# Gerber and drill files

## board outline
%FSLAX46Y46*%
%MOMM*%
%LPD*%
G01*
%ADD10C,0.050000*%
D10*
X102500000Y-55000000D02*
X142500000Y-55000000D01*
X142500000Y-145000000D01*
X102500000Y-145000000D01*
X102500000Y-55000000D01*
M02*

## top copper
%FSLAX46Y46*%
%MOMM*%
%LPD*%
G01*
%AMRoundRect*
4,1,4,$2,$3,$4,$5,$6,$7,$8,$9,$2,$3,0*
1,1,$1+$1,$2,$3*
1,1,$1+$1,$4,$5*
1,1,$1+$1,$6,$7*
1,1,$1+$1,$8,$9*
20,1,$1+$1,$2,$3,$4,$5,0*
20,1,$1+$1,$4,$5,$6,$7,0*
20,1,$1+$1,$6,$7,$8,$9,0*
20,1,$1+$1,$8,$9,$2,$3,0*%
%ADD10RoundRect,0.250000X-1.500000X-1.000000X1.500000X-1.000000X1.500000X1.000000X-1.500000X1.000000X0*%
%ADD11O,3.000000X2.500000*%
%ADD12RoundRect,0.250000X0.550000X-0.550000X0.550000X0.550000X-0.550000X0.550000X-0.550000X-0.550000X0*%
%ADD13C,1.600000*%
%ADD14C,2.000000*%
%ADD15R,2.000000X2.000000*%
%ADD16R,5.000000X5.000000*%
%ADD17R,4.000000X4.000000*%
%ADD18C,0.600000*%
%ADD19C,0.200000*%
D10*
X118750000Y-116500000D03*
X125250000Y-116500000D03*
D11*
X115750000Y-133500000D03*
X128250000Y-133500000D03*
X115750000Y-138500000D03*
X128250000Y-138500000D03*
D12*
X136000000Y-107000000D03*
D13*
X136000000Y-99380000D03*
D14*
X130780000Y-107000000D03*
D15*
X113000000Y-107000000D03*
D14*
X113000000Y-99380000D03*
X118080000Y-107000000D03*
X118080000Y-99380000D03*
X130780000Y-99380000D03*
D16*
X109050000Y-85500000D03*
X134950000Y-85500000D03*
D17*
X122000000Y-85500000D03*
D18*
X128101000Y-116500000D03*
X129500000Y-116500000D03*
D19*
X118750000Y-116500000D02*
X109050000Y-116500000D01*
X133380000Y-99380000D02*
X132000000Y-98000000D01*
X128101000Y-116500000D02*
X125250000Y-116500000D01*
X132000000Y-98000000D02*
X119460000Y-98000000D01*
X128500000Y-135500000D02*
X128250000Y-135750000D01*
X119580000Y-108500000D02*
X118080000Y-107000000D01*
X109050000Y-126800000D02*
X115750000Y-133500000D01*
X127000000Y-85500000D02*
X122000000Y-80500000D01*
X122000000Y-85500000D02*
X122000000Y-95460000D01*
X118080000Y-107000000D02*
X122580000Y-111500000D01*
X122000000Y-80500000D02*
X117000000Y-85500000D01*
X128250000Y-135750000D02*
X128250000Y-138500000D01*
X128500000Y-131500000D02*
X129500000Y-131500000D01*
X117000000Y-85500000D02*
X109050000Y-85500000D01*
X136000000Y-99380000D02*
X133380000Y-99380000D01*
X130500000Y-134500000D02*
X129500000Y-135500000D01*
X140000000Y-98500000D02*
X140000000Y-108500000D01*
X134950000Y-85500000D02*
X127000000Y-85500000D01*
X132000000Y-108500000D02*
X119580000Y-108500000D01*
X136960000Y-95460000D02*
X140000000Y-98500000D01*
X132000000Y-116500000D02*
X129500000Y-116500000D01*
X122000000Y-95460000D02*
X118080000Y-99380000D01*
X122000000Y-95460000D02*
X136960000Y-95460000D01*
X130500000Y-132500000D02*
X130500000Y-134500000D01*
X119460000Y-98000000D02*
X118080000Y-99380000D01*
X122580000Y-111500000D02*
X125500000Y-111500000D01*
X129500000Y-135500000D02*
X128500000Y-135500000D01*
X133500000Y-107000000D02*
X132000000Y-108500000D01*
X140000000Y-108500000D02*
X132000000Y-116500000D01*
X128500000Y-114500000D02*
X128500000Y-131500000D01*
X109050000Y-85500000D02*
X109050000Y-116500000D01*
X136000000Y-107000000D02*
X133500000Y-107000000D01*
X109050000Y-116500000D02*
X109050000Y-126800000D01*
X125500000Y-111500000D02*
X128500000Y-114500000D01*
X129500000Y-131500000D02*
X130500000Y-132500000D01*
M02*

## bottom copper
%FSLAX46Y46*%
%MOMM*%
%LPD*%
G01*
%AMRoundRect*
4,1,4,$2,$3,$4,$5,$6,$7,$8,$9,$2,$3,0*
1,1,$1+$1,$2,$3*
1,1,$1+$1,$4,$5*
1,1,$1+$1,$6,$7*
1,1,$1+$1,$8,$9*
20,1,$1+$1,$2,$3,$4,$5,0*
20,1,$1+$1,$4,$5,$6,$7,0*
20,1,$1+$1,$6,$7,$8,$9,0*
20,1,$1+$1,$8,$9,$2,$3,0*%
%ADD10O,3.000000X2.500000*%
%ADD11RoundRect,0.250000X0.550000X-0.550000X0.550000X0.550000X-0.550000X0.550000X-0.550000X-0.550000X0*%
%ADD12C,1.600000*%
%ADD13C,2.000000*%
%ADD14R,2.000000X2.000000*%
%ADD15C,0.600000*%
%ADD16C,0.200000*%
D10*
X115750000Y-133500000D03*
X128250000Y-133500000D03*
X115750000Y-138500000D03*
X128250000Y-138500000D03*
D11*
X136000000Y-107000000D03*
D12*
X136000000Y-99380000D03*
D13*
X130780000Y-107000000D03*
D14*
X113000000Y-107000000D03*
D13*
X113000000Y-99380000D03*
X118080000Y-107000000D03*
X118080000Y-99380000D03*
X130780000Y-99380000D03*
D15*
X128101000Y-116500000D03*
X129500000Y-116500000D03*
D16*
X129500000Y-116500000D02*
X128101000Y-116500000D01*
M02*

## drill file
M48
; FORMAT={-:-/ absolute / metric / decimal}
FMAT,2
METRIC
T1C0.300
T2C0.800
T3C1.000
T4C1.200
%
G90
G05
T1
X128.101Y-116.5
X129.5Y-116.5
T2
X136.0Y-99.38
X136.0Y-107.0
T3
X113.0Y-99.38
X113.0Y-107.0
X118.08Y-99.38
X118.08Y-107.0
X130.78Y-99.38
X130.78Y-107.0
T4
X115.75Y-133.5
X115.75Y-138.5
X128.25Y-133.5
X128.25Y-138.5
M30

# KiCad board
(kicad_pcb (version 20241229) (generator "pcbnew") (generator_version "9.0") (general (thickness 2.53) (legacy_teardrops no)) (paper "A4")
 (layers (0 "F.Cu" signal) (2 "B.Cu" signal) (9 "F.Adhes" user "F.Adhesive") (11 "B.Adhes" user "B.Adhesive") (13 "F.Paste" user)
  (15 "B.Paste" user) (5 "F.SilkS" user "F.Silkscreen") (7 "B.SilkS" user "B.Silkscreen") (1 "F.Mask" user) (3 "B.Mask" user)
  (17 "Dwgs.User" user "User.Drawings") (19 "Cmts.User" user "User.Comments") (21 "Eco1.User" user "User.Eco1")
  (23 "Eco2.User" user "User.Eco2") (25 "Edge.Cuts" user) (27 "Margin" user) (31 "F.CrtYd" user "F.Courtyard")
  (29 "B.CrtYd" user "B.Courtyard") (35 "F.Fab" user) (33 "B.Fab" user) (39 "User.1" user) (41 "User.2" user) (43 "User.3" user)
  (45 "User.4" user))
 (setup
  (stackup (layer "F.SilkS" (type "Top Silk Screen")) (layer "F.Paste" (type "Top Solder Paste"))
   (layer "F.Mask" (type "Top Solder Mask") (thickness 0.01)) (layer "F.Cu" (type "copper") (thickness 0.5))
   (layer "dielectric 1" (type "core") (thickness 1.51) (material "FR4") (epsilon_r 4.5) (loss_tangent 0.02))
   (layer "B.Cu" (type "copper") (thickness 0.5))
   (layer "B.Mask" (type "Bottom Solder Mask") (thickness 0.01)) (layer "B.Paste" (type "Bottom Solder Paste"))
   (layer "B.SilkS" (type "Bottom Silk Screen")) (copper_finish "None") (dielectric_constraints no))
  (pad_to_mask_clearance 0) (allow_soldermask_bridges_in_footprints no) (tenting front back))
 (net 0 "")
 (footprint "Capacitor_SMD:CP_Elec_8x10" (layer "F.Cu") (at 122 116.5)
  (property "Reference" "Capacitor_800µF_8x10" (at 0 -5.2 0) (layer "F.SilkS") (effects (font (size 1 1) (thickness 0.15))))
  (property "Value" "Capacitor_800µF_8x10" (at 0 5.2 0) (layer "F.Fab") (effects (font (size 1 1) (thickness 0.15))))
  (pad "1" smd roundrect (at -3.25 0) (size 3.5 2.5) (layers "F.Cu" "F.Mask" "F.Paste") (roundrect_rratio 0.1))
  (pad "2" smd roundrect (at 3.25 0) (size 3.5 2.5) (layers "F.Cu" "F.Mask" "F.Paste") (roundrect_rratio 0.1)))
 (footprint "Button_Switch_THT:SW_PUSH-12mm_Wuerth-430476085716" (layer "F.Cu") (at 115.75 133.5)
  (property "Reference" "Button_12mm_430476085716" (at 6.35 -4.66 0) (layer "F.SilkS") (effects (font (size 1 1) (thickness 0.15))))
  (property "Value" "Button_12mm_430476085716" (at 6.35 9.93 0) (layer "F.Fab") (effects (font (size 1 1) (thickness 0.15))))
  (pad "1" thru_hole oval (at 0 0) (size 3 2.5) (drill 1.2) (layers "*.Cu" "*.Mask") (remove_unused_layers no))
  (pad "1" thru_hole oval (at 12.5 0) (size 3 2.5) (drill 1.2) (layers "*.Cu" "*.Mask") (remove_unused_layers no))
  (pad "2" thru_hole oval (at 0 5) (size 3 2.5) (drill 1.2) (layers "*.Cu" "*.Mask") (remove_unused_layers no))
  (pad "2" thru_hole oval (at 12.5 5) (size 3 2.5) (drill 1.2) (layers "*.Cu" "*.Mask") (remove_unused_layers no)))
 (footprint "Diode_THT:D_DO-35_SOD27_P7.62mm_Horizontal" (layer "F.Cu") (at 136 107 90)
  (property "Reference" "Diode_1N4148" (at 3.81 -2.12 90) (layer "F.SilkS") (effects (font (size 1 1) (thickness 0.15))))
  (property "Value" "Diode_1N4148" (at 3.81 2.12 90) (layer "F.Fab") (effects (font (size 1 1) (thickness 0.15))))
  (pad "1" thru_hole roundrect (at 0 0 90) (size 1.6 1.6) (drill 0.8) (layers "*.Cu" "*.Mask") (remove_unused_layers no)
   (roundrect_rratio 0.15625))
  (pad "2" thru_hole circle (at 7.62 0 90) (size 1.6 1.6) (drill 0.8) (layers "*.Cu" "*.Mask") (remove_unused_layers no)))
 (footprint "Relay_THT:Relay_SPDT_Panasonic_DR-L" (layer "F.Cu") (at 113 107)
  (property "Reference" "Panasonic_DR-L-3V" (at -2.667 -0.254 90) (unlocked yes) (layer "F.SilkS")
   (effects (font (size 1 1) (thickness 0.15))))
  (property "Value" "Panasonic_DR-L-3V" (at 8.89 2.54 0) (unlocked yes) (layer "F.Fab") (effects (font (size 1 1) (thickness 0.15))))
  (pad "11" thru_hole circle (at 17.78 0 180) (size 2 2) (drill 1) (layers "*.Cu" "*.Mask") (remove_unused_layers no))
  (pad "12" thru_hole rect (at 0 0 180) (size 2 2) (drill 1) (layers "*.Cu" "*.Mask") (remove_unused_layers no))
  (pad "14" thru_hole circle (at 0 -7.62 180) (size 2 2) (drill 1) (layers "*.Cu" "*.Mask") (remove_unused_layers no))
  (pad "A1" thru_hole circle (at 5.08 0 180) (size 2 2) (drill 1) (layers "*.Cu" "*.Mask") (remove_unused_layers no))
  (pad "A2" thru_hole circle (at 5.08 -7.62 180) (size 2 2) (drill 1) (layers "*.Cu" "*.Mask") (remove_unused_layers no))
  (pad "PE" thru_hole circle (at 17.78 -7.62 180) (size 2 2) (drill 1) (layers "*.Cu" "*.Mask") (remove_unused_layers no)))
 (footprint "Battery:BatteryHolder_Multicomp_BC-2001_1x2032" (layer "F.Cu") (at 122 85.5)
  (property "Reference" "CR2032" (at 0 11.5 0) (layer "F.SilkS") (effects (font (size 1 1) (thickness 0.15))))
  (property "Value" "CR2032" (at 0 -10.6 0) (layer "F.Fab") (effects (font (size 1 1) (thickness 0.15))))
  (pad "1" smd rect (at -12.95 0) (size 5 5) (layers "F.Cu" "F.Mask" "F.Paste"))
  (pad "1" smd rect (at 12.95 0) (size 5 5) (layers "F.Cu" "F.Mask" "F.Paste"))
  (pad "2" smd rect (at 0 0) (size 4 4) (layers "F.Cu" "F.Mask" "F.Paste"))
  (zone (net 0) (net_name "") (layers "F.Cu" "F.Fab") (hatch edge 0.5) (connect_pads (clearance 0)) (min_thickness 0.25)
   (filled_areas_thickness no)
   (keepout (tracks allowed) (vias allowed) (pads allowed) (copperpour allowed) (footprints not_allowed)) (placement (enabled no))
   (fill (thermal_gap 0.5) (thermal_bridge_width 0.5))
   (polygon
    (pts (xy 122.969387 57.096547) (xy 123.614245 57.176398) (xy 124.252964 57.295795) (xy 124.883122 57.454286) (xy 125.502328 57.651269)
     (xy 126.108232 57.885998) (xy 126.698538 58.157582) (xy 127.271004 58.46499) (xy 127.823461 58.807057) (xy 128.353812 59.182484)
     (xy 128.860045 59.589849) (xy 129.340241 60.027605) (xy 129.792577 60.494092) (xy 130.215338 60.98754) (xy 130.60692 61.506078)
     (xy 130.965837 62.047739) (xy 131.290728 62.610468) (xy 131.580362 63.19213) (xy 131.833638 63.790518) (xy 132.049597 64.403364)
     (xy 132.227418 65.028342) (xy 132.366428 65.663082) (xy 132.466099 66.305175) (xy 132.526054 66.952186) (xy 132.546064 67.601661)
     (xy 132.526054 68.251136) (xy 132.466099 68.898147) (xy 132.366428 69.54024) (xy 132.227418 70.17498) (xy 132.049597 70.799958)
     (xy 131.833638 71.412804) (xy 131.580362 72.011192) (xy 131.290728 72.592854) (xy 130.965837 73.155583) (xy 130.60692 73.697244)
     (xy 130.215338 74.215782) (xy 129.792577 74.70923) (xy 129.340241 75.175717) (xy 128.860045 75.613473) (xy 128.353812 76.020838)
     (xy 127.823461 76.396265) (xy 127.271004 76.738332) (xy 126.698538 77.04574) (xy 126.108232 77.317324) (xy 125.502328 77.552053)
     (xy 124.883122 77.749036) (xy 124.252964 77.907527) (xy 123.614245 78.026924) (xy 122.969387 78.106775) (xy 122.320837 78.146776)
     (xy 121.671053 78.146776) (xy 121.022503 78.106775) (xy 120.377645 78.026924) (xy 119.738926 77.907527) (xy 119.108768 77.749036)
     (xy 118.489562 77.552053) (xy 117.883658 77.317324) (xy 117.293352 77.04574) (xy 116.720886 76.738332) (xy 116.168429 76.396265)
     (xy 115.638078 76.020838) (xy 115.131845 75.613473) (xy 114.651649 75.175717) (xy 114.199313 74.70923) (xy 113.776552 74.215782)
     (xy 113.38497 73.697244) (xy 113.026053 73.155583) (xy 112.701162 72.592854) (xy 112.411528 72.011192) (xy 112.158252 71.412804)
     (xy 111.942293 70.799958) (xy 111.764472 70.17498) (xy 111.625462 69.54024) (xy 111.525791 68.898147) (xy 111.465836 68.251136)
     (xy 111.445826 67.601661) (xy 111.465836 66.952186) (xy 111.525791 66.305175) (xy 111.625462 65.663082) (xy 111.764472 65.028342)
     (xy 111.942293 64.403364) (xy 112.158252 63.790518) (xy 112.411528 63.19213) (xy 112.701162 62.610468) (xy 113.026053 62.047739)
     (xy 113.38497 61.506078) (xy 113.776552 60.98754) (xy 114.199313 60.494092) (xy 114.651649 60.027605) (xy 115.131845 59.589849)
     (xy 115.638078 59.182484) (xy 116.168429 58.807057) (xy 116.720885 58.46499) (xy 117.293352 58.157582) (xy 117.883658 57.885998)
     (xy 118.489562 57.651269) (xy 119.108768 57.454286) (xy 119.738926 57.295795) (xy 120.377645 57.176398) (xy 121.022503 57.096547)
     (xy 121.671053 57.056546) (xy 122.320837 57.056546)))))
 (gr_rect (start 102.5 55) (end 142.5 145) (stroke (width 0.05) (type default)) (fill no) (layer "Edge.Cuts"))
 (segment (start 118.75 116.5) (end 109.05 116.5) (width 0.2) (layer "F.Cu") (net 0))
 (segment (start 133.38 99.38) (end 132 98) (width 0.2) (layer "F.Cu") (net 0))
 (segment (start 128.101 116.5) (end 125.25 116.5) (width 0.2) (layer "F.Cu") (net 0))
 (segment (start 132 98) (end 119.46 98) (width 0.2) (layer "F.Cu") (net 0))
 (segment (start 128.5 135.5) (end 128.25 135.75) (width 0.2) (layer "F.Cu") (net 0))
 (segment (start 119.58 108.5) (end 118.08 107) (width 0.2) (layer "F.Cu") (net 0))
 (segment (start 109.05 126.8) (end 115.75 133.5) (width 0.2) (layer "F.Cu") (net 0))
 (segment (start 127 85.5) (end 122 80.5) (width 0.2) (layer "F.Cu") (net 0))
 (segment (start 122 85.5) (end 122 95.46) (width 0.2) (layer "F.Cu") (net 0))
 (segment (start 118.08 107) (end 122.58 111.5) (width 0.2) (layer "F.Cu") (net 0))
 (segment (start 122 80.5) (end 117 85.5) (width 0.2) (layer "F.Cu") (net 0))
 (segment (start 128.25 135.75) (end 128.25 138.5) (width 0.2) (layer "F.Cu") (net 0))
 (segment (start 128.5 131.5) (end 129.5 131.5) (width 0.2) (layer "F.Cu") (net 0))
 (segment (start 117 85.5) (end 109.05 85.5) (width 0.2) (layer "F.Cu") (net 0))
 (segment (start 136 99.38) (end 133.38 99.38) (width 0.2) (layer "F.Cu") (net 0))
 (segment (start 130.5 134.5) (end 129.5 135.5) (width 0.2) (layer "F.Cu") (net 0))
 (segment (start 140 98.5) (end 140 108.5) (width 0.2) (layer "F.Cu") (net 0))
 (segment (start 134.95 85.5) (end 127 85.5) (width 0.2) (layer "F.Cu") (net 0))
 (segment (start 132 108.5) (end 119.58 108.5) (width 0.2) (layer "F.Cu") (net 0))
 (segment (start 136.96 95.46) (end 140 98.5) (width 0.2) (layer "F.Cu") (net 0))
 (segment (start 132 116.5) (end 129.5 116.5) (width 0.2) (layer "F.Cu") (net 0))
 (segment (start 122 95.46) (end 118.08 99.38) (width 0.2) (layer "F.Cu") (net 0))
 (segment (start 122 95.46) (end 136.96 95.46) (width 0.2) (layer "F.Cu") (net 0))
 (segment (start 130.5 132.5) (end 130.5 134.5) (width 0.2) (layer "F.Cu") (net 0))
 (segment (start 119.46 98) (end 118.08 99.38) (width 0.2) (layer "F.Cu") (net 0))
 (segment (start 122.58 111.5) (end 125.5 111.5) (width 0.2) (layer "F.Cu") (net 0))
 (segment (start 129.5 135.5) (end 128.5 135.5) (width 0.2) (layer "F.Cu") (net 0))
 (segment (start 133.5 107) (end 132 108.5) (width 0.2) (layer "F.Cu") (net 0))
 (segment (start 140 108.5) (end 132 116.5) (width 0.2) (layer "F.Cu") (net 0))
 (segment (start 128.5 114.5) (end 128.5 131.5) (width 0.2) (layer "F.Cu") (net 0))
 (segment (start 109.05 85.5) (end 109.05 116.5) (width 0.2) (layer "F.Cu") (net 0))
 (segment (start 136 107) (end 133.5 107) (width 0.2) (layer "F.Cu") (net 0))
 (segment (start 109.05 116.5) (end 109.05 126.8) (width 0.2) (layer "F.Cu") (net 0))
 (segment (start 125.5 111.5) (end 128.5 114.5) (width 0.2) (layer "F.Cu") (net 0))
 (segment (start 129.5 131.5) (end 130.5 132.5) (width 0.2) (layer "F.Cu") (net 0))
 (via (at 128.101 116.5) (size 0.6) (drill 0.3) (layers "F.Cu" "B.Cu") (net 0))
 (via (at 129.5 116.5) (size 0.6) (drill 0.3) (layers "F.Cu" "B.Cu") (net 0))
 (segment (start 129.5 116.5) (end 128.101 116.5) (width 0.2) (layer "B.Cu") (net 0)))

